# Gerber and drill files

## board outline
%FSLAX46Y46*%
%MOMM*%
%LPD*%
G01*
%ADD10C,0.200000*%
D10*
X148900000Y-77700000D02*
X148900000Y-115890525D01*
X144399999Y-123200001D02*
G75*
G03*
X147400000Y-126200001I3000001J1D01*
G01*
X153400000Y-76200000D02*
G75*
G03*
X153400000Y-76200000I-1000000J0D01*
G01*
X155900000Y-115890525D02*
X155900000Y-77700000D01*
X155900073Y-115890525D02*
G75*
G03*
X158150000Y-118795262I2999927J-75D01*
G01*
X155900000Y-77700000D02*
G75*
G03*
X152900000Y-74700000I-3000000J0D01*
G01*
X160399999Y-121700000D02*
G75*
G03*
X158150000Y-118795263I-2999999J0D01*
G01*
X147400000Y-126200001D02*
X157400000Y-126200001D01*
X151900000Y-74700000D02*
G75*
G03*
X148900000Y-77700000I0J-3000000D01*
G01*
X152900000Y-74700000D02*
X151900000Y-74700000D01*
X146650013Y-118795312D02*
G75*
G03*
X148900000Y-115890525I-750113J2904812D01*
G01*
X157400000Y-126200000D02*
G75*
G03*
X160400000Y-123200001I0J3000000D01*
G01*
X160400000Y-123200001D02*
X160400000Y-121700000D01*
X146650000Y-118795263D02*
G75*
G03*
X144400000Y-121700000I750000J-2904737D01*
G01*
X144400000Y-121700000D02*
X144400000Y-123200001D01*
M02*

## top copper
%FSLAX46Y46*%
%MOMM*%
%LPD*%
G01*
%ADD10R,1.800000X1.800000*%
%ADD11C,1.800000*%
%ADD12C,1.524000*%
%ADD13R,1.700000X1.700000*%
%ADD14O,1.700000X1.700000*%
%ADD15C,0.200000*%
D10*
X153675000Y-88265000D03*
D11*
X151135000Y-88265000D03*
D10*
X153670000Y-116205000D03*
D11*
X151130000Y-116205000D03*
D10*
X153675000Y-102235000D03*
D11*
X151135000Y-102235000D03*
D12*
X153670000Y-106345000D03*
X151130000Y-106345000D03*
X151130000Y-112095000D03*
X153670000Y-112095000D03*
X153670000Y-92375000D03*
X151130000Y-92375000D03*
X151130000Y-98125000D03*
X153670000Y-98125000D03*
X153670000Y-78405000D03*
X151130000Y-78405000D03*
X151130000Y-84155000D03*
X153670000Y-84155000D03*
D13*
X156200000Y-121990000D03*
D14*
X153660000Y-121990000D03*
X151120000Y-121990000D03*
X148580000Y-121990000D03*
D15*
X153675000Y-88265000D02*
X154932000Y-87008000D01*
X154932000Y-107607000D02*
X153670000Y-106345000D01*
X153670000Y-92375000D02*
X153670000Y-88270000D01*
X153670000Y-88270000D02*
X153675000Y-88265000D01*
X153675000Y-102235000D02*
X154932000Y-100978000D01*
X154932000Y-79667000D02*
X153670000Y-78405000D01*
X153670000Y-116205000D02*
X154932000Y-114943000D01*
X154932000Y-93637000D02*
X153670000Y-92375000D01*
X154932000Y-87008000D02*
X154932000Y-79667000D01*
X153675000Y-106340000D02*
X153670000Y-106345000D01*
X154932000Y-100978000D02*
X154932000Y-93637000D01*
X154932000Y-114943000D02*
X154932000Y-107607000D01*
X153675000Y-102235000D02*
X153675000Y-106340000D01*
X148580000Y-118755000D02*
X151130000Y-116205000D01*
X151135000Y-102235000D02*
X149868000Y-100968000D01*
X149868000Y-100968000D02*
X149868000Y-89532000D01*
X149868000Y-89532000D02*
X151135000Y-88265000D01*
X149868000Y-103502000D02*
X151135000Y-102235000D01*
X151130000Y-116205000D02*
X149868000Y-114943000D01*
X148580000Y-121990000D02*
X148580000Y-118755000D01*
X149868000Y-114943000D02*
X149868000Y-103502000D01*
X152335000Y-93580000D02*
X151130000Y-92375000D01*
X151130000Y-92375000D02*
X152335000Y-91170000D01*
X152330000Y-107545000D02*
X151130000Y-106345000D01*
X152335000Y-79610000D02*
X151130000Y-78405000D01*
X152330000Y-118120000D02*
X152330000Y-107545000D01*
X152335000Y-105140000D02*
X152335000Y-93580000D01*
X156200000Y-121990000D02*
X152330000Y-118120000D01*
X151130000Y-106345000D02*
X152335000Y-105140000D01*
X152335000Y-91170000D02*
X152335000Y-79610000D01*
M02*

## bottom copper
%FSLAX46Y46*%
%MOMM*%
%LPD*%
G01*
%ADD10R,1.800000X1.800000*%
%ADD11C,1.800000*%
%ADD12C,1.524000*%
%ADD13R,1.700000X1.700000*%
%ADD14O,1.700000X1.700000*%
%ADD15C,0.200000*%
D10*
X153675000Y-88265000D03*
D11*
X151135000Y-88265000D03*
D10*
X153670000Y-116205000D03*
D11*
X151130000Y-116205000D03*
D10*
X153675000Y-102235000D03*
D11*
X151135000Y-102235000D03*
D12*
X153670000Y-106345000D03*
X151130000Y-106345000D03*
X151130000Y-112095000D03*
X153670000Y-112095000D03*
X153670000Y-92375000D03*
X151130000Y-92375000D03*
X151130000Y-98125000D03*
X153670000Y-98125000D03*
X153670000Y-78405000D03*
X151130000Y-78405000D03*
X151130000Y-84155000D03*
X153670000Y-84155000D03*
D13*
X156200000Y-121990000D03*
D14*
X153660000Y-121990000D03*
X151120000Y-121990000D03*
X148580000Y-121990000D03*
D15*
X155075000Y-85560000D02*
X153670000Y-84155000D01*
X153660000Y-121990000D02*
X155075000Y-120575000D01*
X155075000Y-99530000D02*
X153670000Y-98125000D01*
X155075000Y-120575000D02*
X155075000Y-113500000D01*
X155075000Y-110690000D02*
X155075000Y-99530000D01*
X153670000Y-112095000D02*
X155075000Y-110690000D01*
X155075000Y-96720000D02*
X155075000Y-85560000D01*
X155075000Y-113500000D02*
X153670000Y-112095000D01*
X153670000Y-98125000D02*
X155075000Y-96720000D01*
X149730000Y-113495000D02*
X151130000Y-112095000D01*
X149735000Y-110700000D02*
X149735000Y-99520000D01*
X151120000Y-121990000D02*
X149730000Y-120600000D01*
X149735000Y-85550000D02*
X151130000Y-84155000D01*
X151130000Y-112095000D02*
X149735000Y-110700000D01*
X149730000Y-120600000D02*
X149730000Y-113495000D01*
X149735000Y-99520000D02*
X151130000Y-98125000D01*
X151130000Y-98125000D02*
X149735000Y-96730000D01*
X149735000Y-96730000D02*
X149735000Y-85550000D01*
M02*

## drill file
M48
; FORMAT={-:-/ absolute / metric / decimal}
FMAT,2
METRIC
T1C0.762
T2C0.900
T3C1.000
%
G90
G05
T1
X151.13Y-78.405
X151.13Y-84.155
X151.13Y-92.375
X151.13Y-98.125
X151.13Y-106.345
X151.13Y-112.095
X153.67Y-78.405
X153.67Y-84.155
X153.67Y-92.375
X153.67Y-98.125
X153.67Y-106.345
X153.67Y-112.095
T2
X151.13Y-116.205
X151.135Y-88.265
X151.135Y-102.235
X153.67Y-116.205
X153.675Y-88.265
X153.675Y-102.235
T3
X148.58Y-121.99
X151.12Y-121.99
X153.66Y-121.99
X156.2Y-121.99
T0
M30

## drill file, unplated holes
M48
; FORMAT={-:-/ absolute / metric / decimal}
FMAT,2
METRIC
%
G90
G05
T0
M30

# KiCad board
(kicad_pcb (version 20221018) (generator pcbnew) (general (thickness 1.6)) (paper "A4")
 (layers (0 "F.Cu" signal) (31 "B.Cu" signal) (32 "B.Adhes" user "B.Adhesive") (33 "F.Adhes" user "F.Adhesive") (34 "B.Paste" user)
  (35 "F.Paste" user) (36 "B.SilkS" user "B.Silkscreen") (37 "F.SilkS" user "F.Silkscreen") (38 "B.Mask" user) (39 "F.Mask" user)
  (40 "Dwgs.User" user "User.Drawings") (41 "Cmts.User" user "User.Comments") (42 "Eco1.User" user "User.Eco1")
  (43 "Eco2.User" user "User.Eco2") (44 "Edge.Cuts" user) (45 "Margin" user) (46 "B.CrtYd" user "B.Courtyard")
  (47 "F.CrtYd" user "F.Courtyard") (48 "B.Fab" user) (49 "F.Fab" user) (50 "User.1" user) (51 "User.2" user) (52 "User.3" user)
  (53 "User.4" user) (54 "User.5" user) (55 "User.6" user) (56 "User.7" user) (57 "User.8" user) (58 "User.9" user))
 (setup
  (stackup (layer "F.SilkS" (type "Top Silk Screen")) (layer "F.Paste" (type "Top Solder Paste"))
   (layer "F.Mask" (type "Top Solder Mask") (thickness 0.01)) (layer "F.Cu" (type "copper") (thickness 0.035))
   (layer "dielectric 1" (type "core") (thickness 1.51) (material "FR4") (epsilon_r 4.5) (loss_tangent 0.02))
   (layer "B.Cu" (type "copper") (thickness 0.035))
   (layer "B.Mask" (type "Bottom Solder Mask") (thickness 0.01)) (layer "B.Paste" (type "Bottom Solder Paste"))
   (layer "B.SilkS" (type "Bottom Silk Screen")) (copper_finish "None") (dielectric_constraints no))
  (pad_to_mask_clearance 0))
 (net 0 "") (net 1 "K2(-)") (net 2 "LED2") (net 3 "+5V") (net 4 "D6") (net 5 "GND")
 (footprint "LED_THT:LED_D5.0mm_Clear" (layer "F.Cu") (at 153.675 88.265 180)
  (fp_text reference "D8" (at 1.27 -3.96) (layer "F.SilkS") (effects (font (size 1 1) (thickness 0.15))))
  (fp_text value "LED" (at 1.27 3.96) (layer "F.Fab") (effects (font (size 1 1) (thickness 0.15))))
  (pad "1" thru_hole rect (at 0 0 180) (size 1.8 1.8) (drill 0.9) (layers "*.Cu" "*.Mask") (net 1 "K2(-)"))
  (pad "2" thru_hole circle (at 2.54 0 180) (size 1.8 1.8) (drill 0.9) (layers "*.Cu" "*.Mask") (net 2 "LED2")))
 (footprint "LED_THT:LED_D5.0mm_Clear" (layer "F.Cu") (at 153.67 116.205 180)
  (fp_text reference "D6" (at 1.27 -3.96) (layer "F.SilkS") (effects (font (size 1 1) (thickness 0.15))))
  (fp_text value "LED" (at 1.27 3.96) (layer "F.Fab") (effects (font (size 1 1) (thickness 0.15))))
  (pad "1" thru_hole rect (at 0 0 180) (size 1.8 1.8) (drill 0.9) (layers "*.Cu" "*.Mask") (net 1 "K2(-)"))
  (pad "2" thru_hole circle (at 2.54 0 180) (size 1.8 1.8) (drill 0.9) (layers "*.Cu" "*.Mask") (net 2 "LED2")))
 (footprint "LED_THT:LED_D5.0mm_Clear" (layer "F.Cu") (at 153.675 102.235 180)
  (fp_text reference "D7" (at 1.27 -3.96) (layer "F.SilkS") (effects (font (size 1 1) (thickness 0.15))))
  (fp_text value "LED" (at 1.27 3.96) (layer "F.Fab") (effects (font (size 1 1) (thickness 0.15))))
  (pad "1" thru_hole rect (at 0 0 180) (size 1.8 1.8) (drill 0.9) (layers "*.Cu" "*.Mask") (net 1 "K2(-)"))
  (pad "2" thru_hole circle (at 2.54 0 180) (size 1.8 1.8) (drill 0.9) (layers "*.Cu" "*.Mask") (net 2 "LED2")))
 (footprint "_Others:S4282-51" (layer "F.Cu") (at 152.4 109.22 -90)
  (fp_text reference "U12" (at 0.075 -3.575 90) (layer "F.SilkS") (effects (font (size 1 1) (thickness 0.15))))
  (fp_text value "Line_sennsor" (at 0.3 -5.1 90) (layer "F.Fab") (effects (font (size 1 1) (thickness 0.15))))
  (pad "1" thru_hole circle (at -2.875 -1.27 270) (size 1.524 1.524) (drill 0.762) (layers "*.Cu" "*.Mask") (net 1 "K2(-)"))
  (pad "2" thru_hole circle (at -2.875 1.27 270) (size 1.524 1.524) (drill 0.762) (layers "*.Cu" "*.Mask") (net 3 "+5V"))
  (pad "3" thru_hole circle (at 2.875 1.27 270) (size 1.524 1.524) (drill 0.762) (layers "*.Cu" "*.Mask") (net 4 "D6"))
  (pad "4" thru_hole circle (at 2.875 -1.27 270) (size 1.524 1.524) (drill 0.762) (layers "*.Cu" "*.Mask") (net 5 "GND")))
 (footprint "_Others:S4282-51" (layer "F.Cu") (at 152.4 95.25 -90)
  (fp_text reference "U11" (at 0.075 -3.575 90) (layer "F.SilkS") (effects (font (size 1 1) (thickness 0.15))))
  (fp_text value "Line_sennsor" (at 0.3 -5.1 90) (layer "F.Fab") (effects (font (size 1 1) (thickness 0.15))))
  (pad "1" thru_hole circle (at -2.875 -1.27 270) (size 1.524 1.524) (drill 0.762) (layers "*.Cu" "*.Mask") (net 1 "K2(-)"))
  (pad "2" thru_hole circle (at -2.875 1.27 270) (size 1.524 1.524) (drill 0.762) (layers "*.Cu" "*.Mask") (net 3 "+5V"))
  (pad "3" thru_hole circle (at 2.875 1.27 270) (size 1.524 1.524) (drill 0.762) (layers "*.Cu" "*.Mask") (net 4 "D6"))
  (pad "4" thru_hole circle (at 2.875 -1.27 270) (size 1.524 1.524) (drill 0.762) (layers "*.Cu" "*.Mask") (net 5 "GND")))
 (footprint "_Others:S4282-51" (layer "F.Cu") (at 152.4 81.28 -90)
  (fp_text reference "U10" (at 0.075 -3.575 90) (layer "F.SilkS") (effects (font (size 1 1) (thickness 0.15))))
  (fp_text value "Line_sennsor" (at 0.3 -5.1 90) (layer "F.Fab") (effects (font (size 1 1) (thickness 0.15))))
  (pad "1" thru_hole circle (at -2.875 -1.27 270) (size 1.524 1.524) (drill 0.762) (layers "*.Cu" "*.Mask") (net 1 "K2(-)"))
  (pad "2" thru_hole circle (at -2.875 1.27 270) (size 1.524 1.524) (drill 0.762) (layers "*.Cu" "*.Mask") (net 3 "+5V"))
  (pad "3" thru_hole circle (at 2.875 1.27 270) (size 1.524 1.524) (drill 0.762) (layers "*.Cu" "*.Mask") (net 4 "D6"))
  (pad "4" thru_hole circle (at 2.875 -1.27 270) (size 1.524 1.524) (drill 0.762) (layers "*.Cu" "*.Mask") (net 5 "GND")))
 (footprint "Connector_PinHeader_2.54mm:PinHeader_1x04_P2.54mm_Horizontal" (layer "F.Cu") (at 156.2 121.99 -90)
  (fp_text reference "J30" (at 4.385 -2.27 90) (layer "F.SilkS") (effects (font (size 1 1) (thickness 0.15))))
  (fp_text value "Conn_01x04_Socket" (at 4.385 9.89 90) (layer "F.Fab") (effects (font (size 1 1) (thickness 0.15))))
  (pad "1" thru_hole rect (at 0 0 270) (size 1.7 1.7) (drill 1) (layers "*.Cu" "*.Mask") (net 3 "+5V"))
  (pad "2" thru_hole oval (at 0 2.54 270) (size 1.7 1.7) (drill 1) (layers "*.Cu" "*.Mask") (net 5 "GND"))
  (pad "3" thru_hole oval (at 0 5.08 270) (size 1.7 1.7) (drill 1) (layers "*.Cu" "*.Mask") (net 4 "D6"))
  (pad "4" thru_hole oval (at 0 7.62 270) (size 1.7 1.7) (drill 1) (layers "*.Cu" "*.Mask") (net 2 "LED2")))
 (gr_line (start 148.9 77.7) (end 148.9 115.890525) (stroke (width 0.2) (type solid)) (layer "Edge.Cuts"))
 (gr_arc (start 147.4 126.200001) (mid 145.278679 125.321321) (end 144.4 123.200001) (stroke (width 0.2) (type solid)) (layer "Edge.Cuts"))
 (gr_circle (center 152.4 76.2) (end 151.4 76.2) (stroke (width 0.2) (type solid)) (fill none) (layer "Edge.Cuts"))
 (gr_line (start 155.9 115.890525) (end 155.9 77.7) (stroke (width 0.2) (type solid)) (layer "Edge.Cuts"))
 (gr_arc (start 158.15 118.795263) (mid 156.528282 117.727645) (end 155.9 115.890525) (stroke (width 0.2) (type solid)) (layer "Edge.Cuts"))
 (gr_arc (start 152.9 74.7) (mid 155.02132 75.57868) (end 155.9 77.7) (stroke (width 0.2) (type solid)) (layer "Edge.Cuts"))
 (gr_arc (start 158.15 118.795263) (mid 159.771708 119.862883) (end 160.4 121.7) (stroke (width 0.2) (type solid)) (layer "Edge.Cuts"))
 (gr_line (start 147.4 126.200001) (end 157.4 126.200001) (stroke (width 0.2) (type solid)) (layer "Edge.Cuts"))
 (gr_arc (start 148.9 77.7) (mid 149.77868 75.57868) (end 151.9 74.7) (stroke (width 0.2) (type solid)) (layer "Edge.Cuts"))
 (gr_line (start 152.9 74.7) (end 151.9 74.7) (stroke (width 0.2) (type solid)) (layer "Edge.Cuts"))
 (gr_arc (start 148.9 115.890525) (mid 148.271699 117.72763) (end 146.65 118.795263) (stroke (width 0.2) (type solid)) (layer "Edge.Cuts"))
 (gr_arc (start 160.4 123.200001) (mid 159.52132 125.321321) (end 157.4 126.200001) (stroke (width 0.2) (type solid)) (layer "Edge.Cuts"))
 (gr_line (start 160.4 123.200001) (end 160.4 121.7) (stroke (width 0.2) (type solid)) (layer "Edge.Cuts"))
 (gr_arc (start 144.4 121.7) (mid 145.028292 119.862883) (end 146.65 118.795263) (stroke (width 0.2) (type solid)) (layer "Edge.Cuts"))
 (gr_line (start 144.4 121.7) (end 144.4 123.200001) (stroke (width 0.2) (type solid)) (layer "Edge.Cuts"))
 (segment (start 153.675 88.265) (end 154.932 87.008) (width 0.2) (layer "F.Cu") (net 1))
 (segment (start 154.932 107.607) (end 153.67 106.345) (width 0.2) (layer "F.Cu") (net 1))
 (segment (start 153.67 92.375) (end 153.67 88.27) (width 0.2) (layer "F.Cu") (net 1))
 (segment (start 153.67 88.27) (end 153.675 88.265) (width 0.2) (layer "F.Cu") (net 1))
 (segment (start 153.675 102.235) (end 154.932 100.978) (width 0.2) (layer "F.Cu") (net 1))
 (segment (start 154.932 79.667) (end 153.67 78.405) (width 0.2) (layer "F.Cu") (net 1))
 (segment (start 153.67 116.205) (end 154.932 114.943) (width 0.2) (layer "F.Cu") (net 1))
 (segment (start 154.932 93.637) (end 153.67 92.375) (width 0.2) (layer "F.Cu") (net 1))
 (segment (start 154.932 87.008) (end 154.932 79.667) (width 0.2) (layer "F.Cu") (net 1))
 (segment (start 153.675 106.34) (end 153.67 106.345) (width 0.2) (layer "F.Cu") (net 1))
 (segment (start 154.932 100.978) (end 154.932 93.637) (width 0.2) (layer "F.Cu") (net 1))
 (segment (start 154.932 114.943) (end 154.932 107.607) (width 0.2) (layer "F.Cu") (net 1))
 (segment (start 153.675 102.235) (end 153.675 106.34) (width 0.2) (layer "F.Cu") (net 1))
 (segment (start 148.58 118.755) (end 151.13 116.205) (width 0.2) (layer "F.Cu") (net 2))
 (segment (start 151.135 102.235) (end 149.868 100.968) (width 0.2) (layer "F.Cu") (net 2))
 (segment (start 149.868 100.968) (end 149.868 89.532) (width 0.2) (layer "F.Cu") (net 2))
 (segment (start 149.868 89.532) (end 151.135 88.265) (width 0.2) (layer "F.Cu") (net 2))
 (segment (start 149.868 103.502) (end 151.135 102.235) (width 0.2) (layer "F.Cu") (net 2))
 (segment (start 151.13 116.205) (end 149.868 114.943) (width 0.2) (layer "F.Cu") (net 2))
 (segment (start 148.58 121.99) (end 148.58 118.755) (width 0.2) (layer "F.Cu") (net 2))
 (segment (start 149.868 114.943) (end 149.868 103.502) (width 0.2) (layer "F.Cu") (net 2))
 (segment (start 152.335 93.58) (end 151.13 92.375) (width 0.2) (layer "F.Cu") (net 3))
 (segment (start 151.13 92.375) (end 152.335 91.17) (width 0.2) (layer "F.Cu") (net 3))
 (segment (start 152.33 107.545) (end 151.13 106.345) (width 0.2) (layer "F.Cu") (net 3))
 (segment (start 152.335 79.61) (end 151.13 78.405) (width 0.2) (layer "F.Cu") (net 3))
 (segment (start 152.33 118.12) (end 152.33 107.545) (width 0.2) (layer "F.Cu") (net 3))
 (segment (start 152.335 105.14) (end 152.335 93.58) (width 0.2) (layer "F.Cu") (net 3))
 (segment (start 156.2 121.99) (end 152.33 118.12) (width 0.2) (layer "F.Cu") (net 3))
 (segment (start 151.13 106.345) (end 152.335 105.14) (width 0.2) (layer "F.Cu") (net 3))
 (segment (start 152.335 91.17) (end 152.335 79.61) (width 0.2) (layer "F.Cu") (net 3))
 (segment (start 155.075 85.56) (end 153.67 84.155) (width 0.2) (layer "B.Cu") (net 5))
 (segment (start 153.66 121.99) (end 155.075 120.575) (width 0.2) (layer "B.Cu") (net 5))
 (segment (start 155.075 99.53) (end 153.67 98.125) (width 0.2) (layer "B.Cu") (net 5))
 (segment (start 155.075 120.575) (end 155.075 113.5) (width 0.2) (layer "B.Cu") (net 5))
 (segment (start 155.075 110.69) (end 155.075 99.53) (width 0.2) (layer "B.Cu") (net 5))
 (segment (start 153.67 112.095) (end 155.075 110.69) (width 0.2) (layer "B.Cu") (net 5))
 (segment (start 155.075 96.72) (end 155.075 85.56) (width 0.2) (layer "B.Cu") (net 5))
 (segment (start 155.075 113.5) (end 153.67 112.095) (width 0.2) (layer "B.Cu") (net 5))
 (segment (start 153.67 98.125) (end 155.075 96.72) (width 0.2) (layer "B.Cu") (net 5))
 (segment (start 149.73 113.495) (end 151.13 112.095) (width 0.2) (layer "B.Cu") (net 4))
 (segment (start 149.735 110.7) (end 149.735 99.52) (width 0.2) (layer "B.Cu") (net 4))
 (segment (start 151.12 121.99) (end 149.73 120.6) (width 0.2) (layer "B.Cu") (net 4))
 (segment (start 149.735 85.55) (end 151.13 84.155) (width 0.2) (layer "B.Cu") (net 4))
 (segment (start 151.13 112.095) (end 149.735 110.7) (width 0.2) (layer "B.Cu") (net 4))
 (segment (start 149.73 120.6) (end 149.73 113.495) (width 0.2) (layer "B.Cu") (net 4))
 (segment (start 149.735 99.52) (end 151.13 98.125) (width 0.2) (layer "B.Cu") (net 4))
 (segment (start 151.13 98.125) (end 149.735 96.73) (width 0.2) (layer "B.Cu") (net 4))
 (segment (start 149.735 96.73) (end 149.735 85.55) (width 0.2) (layer "B.Cu") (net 4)))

